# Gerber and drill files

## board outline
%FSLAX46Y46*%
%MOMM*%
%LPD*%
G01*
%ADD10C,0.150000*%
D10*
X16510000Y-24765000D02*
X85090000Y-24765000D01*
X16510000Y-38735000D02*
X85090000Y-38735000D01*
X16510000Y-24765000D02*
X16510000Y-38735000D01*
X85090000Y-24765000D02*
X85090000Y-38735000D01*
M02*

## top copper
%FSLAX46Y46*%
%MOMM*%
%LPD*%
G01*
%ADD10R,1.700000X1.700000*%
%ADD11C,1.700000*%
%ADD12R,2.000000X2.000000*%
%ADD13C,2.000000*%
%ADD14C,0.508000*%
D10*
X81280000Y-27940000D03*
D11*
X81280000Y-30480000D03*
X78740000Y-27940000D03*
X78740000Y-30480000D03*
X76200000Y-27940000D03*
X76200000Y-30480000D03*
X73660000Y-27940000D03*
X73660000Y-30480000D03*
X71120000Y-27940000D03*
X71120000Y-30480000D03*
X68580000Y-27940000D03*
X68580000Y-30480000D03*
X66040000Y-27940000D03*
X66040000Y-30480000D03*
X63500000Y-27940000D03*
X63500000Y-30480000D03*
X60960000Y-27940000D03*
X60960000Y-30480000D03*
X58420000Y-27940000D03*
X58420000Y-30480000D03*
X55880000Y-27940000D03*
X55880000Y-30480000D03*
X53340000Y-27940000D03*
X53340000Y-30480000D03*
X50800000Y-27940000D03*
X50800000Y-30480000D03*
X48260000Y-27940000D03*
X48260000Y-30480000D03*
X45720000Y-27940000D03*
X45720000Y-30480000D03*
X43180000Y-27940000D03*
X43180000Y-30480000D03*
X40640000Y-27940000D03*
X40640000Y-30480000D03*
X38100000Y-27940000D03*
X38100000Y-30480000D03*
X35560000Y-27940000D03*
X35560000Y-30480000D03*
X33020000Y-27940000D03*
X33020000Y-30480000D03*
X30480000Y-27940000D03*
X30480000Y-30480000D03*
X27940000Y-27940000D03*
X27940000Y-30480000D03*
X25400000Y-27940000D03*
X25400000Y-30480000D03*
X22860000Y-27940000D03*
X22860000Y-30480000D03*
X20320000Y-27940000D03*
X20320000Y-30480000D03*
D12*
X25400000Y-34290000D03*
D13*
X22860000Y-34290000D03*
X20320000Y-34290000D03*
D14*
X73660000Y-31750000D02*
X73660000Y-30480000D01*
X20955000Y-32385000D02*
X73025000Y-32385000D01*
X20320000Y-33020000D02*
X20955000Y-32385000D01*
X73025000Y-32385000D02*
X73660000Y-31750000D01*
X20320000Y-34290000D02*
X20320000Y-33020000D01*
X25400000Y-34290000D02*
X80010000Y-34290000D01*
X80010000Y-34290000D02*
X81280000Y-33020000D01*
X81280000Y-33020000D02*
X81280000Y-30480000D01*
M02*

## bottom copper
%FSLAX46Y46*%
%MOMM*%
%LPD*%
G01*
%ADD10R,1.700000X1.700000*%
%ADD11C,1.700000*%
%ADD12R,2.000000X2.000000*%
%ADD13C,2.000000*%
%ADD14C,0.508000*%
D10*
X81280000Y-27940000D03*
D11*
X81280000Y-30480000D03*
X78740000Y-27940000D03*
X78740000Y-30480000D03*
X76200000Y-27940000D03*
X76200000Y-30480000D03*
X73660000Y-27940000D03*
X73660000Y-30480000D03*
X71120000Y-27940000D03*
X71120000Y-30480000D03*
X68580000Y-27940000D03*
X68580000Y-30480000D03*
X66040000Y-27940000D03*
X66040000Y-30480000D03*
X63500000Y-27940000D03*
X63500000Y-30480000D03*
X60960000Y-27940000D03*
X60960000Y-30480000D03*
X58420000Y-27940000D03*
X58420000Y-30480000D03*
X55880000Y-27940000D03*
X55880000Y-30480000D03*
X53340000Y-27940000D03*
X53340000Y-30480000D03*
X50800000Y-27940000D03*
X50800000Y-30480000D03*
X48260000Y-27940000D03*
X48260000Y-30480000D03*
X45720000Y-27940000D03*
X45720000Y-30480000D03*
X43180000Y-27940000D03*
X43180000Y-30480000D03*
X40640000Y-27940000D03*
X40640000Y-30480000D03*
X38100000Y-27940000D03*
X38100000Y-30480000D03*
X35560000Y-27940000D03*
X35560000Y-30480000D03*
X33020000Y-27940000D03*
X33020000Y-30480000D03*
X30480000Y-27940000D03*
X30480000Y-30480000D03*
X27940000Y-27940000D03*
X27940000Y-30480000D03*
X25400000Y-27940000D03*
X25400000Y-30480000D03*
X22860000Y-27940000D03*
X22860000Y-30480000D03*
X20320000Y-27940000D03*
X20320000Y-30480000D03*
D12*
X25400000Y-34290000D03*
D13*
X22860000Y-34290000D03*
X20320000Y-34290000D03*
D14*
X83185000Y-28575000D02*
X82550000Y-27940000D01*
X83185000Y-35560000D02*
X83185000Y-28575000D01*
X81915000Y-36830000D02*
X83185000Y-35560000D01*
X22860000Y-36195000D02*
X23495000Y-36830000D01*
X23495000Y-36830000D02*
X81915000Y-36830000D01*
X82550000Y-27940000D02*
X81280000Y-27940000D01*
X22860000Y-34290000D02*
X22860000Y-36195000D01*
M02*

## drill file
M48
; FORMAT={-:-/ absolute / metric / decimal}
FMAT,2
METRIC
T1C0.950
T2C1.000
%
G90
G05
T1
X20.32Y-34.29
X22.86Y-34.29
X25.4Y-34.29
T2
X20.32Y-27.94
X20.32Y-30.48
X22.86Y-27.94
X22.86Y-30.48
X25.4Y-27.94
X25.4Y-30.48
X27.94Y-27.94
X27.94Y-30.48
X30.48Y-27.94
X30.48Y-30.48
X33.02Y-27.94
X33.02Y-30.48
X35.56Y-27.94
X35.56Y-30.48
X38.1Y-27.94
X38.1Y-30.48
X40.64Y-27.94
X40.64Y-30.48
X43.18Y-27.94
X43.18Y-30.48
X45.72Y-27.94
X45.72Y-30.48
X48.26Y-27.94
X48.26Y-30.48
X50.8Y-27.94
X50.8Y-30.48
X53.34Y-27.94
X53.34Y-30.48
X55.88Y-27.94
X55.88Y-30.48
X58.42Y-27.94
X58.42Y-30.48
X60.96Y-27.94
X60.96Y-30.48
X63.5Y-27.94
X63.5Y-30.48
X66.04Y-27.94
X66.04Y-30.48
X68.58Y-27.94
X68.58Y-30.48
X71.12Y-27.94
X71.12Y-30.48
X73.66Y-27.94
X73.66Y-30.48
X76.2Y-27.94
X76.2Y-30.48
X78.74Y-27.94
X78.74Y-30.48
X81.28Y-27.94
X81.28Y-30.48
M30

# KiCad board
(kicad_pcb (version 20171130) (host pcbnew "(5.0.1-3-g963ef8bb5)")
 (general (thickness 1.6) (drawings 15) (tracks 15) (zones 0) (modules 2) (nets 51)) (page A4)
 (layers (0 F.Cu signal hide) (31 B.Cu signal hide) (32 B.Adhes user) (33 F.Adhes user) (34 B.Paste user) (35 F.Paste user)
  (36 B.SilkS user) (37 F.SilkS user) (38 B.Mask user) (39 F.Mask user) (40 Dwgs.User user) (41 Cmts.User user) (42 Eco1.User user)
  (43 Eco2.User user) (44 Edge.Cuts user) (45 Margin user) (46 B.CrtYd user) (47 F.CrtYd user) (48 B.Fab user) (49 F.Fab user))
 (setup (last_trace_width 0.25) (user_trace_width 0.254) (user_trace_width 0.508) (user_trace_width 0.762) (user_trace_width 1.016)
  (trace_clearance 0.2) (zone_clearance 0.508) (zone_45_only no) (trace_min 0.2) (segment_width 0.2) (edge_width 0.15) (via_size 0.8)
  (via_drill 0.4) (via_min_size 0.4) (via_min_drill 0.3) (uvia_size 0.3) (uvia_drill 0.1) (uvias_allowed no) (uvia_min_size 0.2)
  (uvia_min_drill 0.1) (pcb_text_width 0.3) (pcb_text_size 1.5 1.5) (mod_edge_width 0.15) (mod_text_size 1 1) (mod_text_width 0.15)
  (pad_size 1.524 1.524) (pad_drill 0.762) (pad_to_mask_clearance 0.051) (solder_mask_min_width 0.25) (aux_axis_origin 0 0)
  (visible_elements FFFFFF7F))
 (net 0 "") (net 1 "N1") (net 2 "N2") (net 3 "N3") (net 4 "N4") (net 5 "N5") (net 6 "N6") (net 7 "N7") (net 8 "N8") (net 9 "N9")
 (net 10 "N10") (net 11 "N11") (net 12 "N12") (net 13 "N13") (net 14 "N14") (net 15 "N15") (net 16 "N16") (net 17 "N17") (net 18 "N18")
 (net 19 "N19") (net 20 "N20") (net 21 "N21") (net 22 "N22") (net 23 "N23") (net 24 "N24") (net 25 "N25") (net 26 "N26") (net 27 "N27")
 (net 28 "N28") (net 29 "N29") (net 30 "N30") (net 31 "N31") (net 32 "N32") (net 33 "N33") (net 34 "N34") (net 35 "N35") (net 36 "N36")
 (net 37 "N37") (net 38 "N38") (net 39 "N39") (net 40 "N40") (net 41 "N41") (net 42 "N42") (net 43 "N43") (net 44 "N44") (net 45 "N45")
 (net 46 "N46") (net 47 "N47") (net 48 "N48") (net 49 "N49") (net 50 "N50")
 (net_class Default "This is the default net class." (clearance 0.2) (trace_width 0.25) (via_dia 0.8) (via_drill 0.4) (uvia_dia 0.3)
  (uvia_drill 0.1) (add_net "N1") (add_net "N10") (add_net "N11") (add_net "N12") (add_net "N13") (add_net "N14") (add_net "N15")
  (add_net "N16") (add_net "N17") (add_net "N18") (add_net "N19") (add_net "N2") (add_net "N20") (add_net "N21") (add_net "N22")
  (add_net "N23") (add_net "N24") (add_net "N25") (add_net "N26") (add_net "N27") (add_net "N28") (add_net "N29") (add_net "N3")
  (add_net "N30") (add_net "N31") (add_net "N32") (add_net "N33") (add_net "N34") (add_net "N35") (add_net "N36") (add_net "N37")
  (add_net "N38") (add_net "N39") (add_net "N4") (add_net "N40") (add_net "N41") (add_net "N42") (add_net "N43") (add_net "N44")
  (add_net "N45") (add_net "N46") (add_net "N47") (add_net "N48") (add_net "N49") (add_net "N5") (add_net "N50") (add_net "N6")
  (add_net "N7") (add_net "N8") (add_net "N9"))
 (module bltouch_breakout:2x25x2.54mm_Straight (layer F.Cu) (at 81.28 27.94 180)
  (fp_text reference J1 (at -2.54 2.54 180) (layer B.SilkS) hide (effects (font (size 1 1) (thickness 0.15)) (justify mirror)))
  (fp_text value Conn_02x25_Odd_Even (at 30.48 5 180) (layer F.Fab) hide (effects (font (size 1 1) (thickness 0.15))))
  (pad 1 thru_hole rect (at 0 0 180) (size 1.7 1.7) (drill 1) (layers *.Cu *.Mask) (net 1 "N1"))
  (pad 2 thru_hole circle (at 0 -2.54 180) (size 1.7 1.7) (drill 1) (layers *.Cu *.Mask) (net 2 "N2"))
  (pad 3 thru_hole circle (at 2.54 0 180) (size 1.7 1.7) (drill 1) (layers *.Cu *.Mask) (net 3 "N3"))
  (pad 4 thru_hole circle (at 2.54 -2.54 180) (size 1.7 1.7) (drill 1) (layers *.Cu *.Mask) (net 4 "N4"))
  (pad 5 thru_hole circle (at 5.08 0 180) (size 1.7 1.7) (drill 1) (layers *.Cu *.Mask) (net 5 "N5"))
  (pad 6 thru_hole circle (at 5.08 -2.54 180) (size 1.7 1.7) (drill 1) (layers *.Cu *.Mask) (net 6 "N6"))
  (pad 7 thru_hole circle (at 7.62 0 180) (size 1.7 1.7) (drill 1) (layers *.Cu *.Mask) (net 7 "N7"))
  (pad 8 thru_hole circle (at 7.62 -2.54 180) (size 1.7 1.7) (drill 1) (layers *.Cu *.Mask) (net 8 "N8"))
  (pad 9 thru_hole circle (at 10.16 0 180) (size 1.7 1.7) (drill 1) (layers *.Cu *.Mask) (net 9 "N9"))
  (pad 10 thru_hole circle (at 10.16 -2.54 180) (size 1.7 1.7) (drill 1) (layers *.Cu *.Mask) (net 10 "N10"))
  (pad 11 thru_hole circle (at 12.7 0 180) (size 1.7 1.7) (drill 1) (layers *.Cu *.Mask) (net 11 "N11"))
  (pad 12 thru_hole circle (at 12.7 -2.54 180) (size 1.7 1.7) (drill 1) (layers *.Cu *.Mask) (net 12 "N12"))
  (pad 13 thru_hole circle (at 15.24 0 180) (size 1.7 1.7) (drill 1) (layers *.Cu *.Mask) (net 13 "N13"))
  (pad 14 thru_hole circle (at 15.24 -2.54 180) (size 1.7 1.7) (drill 1) (layers *.Cu *.Mask) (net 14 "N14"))
  (pad 15 thru_hole circle (at 17.78 0 180) (size 1.7 1.7) (drill 1) (layers *.Cu *.Mask) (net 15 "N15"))
  (pad 16 thru_hole circle (at 17.78 -2.54 180) (size 1.7 1.7) (drill 1) (layers *.Cu *.Mask) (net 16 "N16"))
  (pad 17 thru_hole circle (at 20.32 0 180) (size 1.7 1.7) (drill 1) (layers *.Cu *.Mask) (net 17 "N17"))
  (pad 18 thru_hole circle (at 20.32 -2.54 180) (size 1.7 1.7) (drill 1) (layers *.Cu *.Mask) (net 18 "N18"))
  (pad 19 thru_hole circle (at 22.86 0 180) (size 1.7 1.7) (drill 1) (layers *.Cu *.Mask) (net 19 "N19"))
  (pad 20 thru_hole circle (at 22.86 -2.54 180) (size 1.7 1.7) (drill 1) (layers *.Cu *.Mask) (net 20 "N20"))
  (pad 21 thru_hole circle (at 25.4 0 180) (size 1.7 1.7) (drill 1) (layers *.Cu *.Mask) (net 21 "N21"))
  (pad 22 thru_hole circle (at 25.4 -2.54 180) (size 1.7 1.7) (drill 1) (layers *.Cu *.Mask) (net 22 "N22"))
  (pad 23 thru_hole circle (at 27.94 0 180) (size 1.7 1.7) (drill 1) (layers *.Cu *.Mask) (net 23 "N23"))
  (pad 24 thru_hole circle (at 27.94 -2.54 180) (size 1.7 1.7) (drill 1) (layers *.Cu *.Mask) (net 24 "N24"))
  (pad 25 thru_hole circle (at 30.48 0 180) (size 1.7 1.7) (drill 1) (layers *.Cu *.Mask) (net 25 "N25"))
  (pad 26 thru_hole circle (at 30.48 -2.54 180) (size 1.7 1.7) (drill 1) (layers *.Cu *.Mask) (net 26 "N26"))
  (pad 27 thru_hole circle (at 33.02 0 180) (size 1.7 1.7) (drill 1) (layers *.Cu *.Mask) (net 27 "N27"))
  (pad 28 thru_hole circle (at 33.02 -2.54 180) (size 1.7 1.7) (drill 1) (layers *.Cu *.Mask) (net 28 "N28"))
  (pad 29 thru_hole circle (at 35.56 0 180) (size 1.7 1.7) (drill 1) (layers *.Cu *.Mask) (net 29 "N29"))
  (pad 30 thru_hole circle (at 35.56 -2.54 180) (size 1.7 1.7) (drill 1) (layers *.Cu *.Mask) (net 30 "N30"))
  (pad 31 thru_hole circle (at 38.1 0 180) (size 1.7 1.7) (drill 1) (layers *.Cu *.Mask) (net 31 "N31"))
  (pad 32 thru_hole circle (at 38.1 -2.54 180) (size 1.7 1.7) (drill 1) (layers *.Cu *.Mask) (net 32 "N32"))
  (pad 33 thru_hole circle (at 40.64 0 180) (size 1.7 1.7) (drill 1) (layers *.Cu *.Mask) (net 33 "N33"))
  (pad 34 thru_hole circle (at 40.64 -2.54 180) (size 1.7 1.7) (drill 1) (layers *.Cu *.Mask) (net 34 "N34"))
  (pad 35 thru_hole circle (at 43.18 0 180) (size 1.7 1.7) (drill 1) (layers *.Cu *.Mask) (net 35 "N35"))
  (pad 36 thru_hole circle (at 43.18 -2.54 180) (size 1.7 1.7) (drill 1) (layers *.Cu *.Mask) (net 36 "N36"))
  (pad 37 thru_hole circle (at 45.72 0 180) (size 1.7 1.7) (drill 1) (layers *.Cu *.Mask) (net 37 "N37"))
  (pad 38 thru_hole circle (at 45.72 -2.54 180) (size 1.7 1.7) (drill 1) (layers *.Cu *.Mask) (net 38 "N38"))
  (pad 39 thru_hole circle (at 48.26 0 180) (size 1.7 1.7) (drill 1) (layers *.Cu *.Mask) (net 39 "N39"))
  (pad 40 thru_hole circle (at 48.26 -2.54 180) (size 1.7 1.7) (drill 1) (layers *.Cu *.Mask) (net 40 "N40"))
  (pad 41 thru_hole circle (at 50.8 0 180) (size 1.7 1.7) (drill 1) (layers *.Cu *.Mask) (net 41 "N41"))
  (pad 42 thru_hole circle (at 50.8 -2.54 180) (size 1.7 1.7) (drill 1) (layers *.Cu *.Mask) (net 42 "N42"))
  (pad 43 thru_hole circle (at 53.34 0 180) (size 1.7 1.7) (drill 1) (layers *.Cu *.Mask) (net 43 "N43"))
  (pad 44 thru_hole circle (at 53.34 -2.54 180) (size 1.7 1.7) (drill 1) (layers *.Cu *.Mask) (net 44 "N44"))
  (pad 45 thru_hole circle (at 55.88 0 180) (size 1.7 1.7) (drill 1) (layers *.Cu *.Mask) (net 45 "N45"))
  (pad 46 thru_hole circle (at 55.88 -2.54 180) (size 1.7 1.7) (drill 1) (layers *.Cu *.Mask) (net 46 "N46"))
  (pad 47 thru_hole circle (at 58.42 0 180) (size 1.7 1.7) (drill 1) (layers *.Cu *.Mask) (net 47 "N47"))
  (pad 48 thru_hole circle (at 58.42 -2.54 180) (size 1.7 1.7) (drill 1) (layers *.Cu *.Mask) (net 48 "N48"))
  (pad 49 thru_hole circle (at 60.96 0 180) (size 1.7 1.7) (drill 1) (layers *.Cu *.Mask) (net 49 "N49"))
  (pad 50 thru_hole circle (at 60.96 -2.54 180) (size 1.7 1.7) (drill 1) (layers *.Cu *.Mask) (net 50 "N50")))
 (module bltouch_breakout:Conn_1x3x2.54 (layer F.Cu) (at 25.4 34.29 270)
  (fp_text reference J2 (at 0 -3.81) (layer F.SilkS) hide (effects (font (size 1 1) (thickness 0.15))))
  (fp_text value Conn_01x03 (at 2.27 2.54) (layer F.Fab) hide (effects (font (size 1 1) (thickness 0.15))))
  (pad 1 thru_hole rect (at 0 0 270) (size 2 2) (drill 0.95) (layers *.Cu *.Mask) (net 2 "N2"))
  (pad 2 thru_hole circle (at 0 2.54 270) (size 2 2) (drill 0.95) (layers *.Cu *.Mask) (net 1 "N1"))
  (pad 3 thru_hole circle (at 0 5.08 270) (size 2 2) (drill 0.95) (layers *.Cu *.Mask) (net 8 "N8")))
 (gr_line (start 16.51 24.765) (end 85.09 24.765) (layer Edge.Cuts) (width 0.15))
 (gr_line (start 16.51 38.735) (end 85.09 38.735) (layer Edge.Cuts) (width 0.15))
 (gr_line (start 16.51 24.765) (end 16.51 38.735) (layer Edge.Cuts) (width 0.15))
 (gr_line (start 85.09 24.765) (end 85.09 38.735) (layer Edge.Cuts) (width 0.15))
 (segment (start 73.66 31.75) (end 73.66 30.48) (width 0.508) (layer F.Cu) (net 8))
 (segment (start 20.955 32.385) (end 73.025 32.385) (width 0.508) (layer F.Cu) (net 8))
 (segment (start 20.32 33.02) (end 20.955 32.385) (width 0.508) (layer F.Cu) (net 8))
 (segment (start 73.025 32.385) (end 73.66 31.75) (width 0.508) (layer F.Cu) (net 8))
 (segment (start 20.32 34.29) (end 20.32 33.02) (width 0.508) (layer F.Cu) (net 8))
 (segment (start 25.4 34.29) (end 80.01 34.29) (width 0.508) (layer F.Cu) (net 2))
 (segment (start 80.01 34.29) (end 81.28 33.02) (width 0.508) (layer F.Cu) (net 2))
 (segment (start 81.28 33.02) (end 81.28 30.48) (width 0.508) (layer F.Cu) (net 2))
 (segment (start 83.185 28.575) (end 82.55 27.94) (width 0.508) (layer B.Cu) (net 1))
 (segment (start 83.185 35.56) (end 83.185 28.575) (width 0.508) (layer B.Cu) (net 1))
 (segment (start 81.915 36.83) (end 83.185 35.56) (width 0.508) (layer B.Cu) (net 1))
 (segment (start 22.86 36.195) (end 23.495 36.83) (width 0.508) (layer B.Cu) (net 1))
 (segment (start 23.495 36.83) (end 81.915 36.83) (width 0.508) (layer B.Cu) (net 1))
 (segment (start 82.55 27.94) (end 81.28 27.94) (width 0.508) (layer B.Cu) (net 1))
 (segment (start 22.86 34.29) (end 22.86 36.195) (width 0.508) (layer B.Cu) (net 1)))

